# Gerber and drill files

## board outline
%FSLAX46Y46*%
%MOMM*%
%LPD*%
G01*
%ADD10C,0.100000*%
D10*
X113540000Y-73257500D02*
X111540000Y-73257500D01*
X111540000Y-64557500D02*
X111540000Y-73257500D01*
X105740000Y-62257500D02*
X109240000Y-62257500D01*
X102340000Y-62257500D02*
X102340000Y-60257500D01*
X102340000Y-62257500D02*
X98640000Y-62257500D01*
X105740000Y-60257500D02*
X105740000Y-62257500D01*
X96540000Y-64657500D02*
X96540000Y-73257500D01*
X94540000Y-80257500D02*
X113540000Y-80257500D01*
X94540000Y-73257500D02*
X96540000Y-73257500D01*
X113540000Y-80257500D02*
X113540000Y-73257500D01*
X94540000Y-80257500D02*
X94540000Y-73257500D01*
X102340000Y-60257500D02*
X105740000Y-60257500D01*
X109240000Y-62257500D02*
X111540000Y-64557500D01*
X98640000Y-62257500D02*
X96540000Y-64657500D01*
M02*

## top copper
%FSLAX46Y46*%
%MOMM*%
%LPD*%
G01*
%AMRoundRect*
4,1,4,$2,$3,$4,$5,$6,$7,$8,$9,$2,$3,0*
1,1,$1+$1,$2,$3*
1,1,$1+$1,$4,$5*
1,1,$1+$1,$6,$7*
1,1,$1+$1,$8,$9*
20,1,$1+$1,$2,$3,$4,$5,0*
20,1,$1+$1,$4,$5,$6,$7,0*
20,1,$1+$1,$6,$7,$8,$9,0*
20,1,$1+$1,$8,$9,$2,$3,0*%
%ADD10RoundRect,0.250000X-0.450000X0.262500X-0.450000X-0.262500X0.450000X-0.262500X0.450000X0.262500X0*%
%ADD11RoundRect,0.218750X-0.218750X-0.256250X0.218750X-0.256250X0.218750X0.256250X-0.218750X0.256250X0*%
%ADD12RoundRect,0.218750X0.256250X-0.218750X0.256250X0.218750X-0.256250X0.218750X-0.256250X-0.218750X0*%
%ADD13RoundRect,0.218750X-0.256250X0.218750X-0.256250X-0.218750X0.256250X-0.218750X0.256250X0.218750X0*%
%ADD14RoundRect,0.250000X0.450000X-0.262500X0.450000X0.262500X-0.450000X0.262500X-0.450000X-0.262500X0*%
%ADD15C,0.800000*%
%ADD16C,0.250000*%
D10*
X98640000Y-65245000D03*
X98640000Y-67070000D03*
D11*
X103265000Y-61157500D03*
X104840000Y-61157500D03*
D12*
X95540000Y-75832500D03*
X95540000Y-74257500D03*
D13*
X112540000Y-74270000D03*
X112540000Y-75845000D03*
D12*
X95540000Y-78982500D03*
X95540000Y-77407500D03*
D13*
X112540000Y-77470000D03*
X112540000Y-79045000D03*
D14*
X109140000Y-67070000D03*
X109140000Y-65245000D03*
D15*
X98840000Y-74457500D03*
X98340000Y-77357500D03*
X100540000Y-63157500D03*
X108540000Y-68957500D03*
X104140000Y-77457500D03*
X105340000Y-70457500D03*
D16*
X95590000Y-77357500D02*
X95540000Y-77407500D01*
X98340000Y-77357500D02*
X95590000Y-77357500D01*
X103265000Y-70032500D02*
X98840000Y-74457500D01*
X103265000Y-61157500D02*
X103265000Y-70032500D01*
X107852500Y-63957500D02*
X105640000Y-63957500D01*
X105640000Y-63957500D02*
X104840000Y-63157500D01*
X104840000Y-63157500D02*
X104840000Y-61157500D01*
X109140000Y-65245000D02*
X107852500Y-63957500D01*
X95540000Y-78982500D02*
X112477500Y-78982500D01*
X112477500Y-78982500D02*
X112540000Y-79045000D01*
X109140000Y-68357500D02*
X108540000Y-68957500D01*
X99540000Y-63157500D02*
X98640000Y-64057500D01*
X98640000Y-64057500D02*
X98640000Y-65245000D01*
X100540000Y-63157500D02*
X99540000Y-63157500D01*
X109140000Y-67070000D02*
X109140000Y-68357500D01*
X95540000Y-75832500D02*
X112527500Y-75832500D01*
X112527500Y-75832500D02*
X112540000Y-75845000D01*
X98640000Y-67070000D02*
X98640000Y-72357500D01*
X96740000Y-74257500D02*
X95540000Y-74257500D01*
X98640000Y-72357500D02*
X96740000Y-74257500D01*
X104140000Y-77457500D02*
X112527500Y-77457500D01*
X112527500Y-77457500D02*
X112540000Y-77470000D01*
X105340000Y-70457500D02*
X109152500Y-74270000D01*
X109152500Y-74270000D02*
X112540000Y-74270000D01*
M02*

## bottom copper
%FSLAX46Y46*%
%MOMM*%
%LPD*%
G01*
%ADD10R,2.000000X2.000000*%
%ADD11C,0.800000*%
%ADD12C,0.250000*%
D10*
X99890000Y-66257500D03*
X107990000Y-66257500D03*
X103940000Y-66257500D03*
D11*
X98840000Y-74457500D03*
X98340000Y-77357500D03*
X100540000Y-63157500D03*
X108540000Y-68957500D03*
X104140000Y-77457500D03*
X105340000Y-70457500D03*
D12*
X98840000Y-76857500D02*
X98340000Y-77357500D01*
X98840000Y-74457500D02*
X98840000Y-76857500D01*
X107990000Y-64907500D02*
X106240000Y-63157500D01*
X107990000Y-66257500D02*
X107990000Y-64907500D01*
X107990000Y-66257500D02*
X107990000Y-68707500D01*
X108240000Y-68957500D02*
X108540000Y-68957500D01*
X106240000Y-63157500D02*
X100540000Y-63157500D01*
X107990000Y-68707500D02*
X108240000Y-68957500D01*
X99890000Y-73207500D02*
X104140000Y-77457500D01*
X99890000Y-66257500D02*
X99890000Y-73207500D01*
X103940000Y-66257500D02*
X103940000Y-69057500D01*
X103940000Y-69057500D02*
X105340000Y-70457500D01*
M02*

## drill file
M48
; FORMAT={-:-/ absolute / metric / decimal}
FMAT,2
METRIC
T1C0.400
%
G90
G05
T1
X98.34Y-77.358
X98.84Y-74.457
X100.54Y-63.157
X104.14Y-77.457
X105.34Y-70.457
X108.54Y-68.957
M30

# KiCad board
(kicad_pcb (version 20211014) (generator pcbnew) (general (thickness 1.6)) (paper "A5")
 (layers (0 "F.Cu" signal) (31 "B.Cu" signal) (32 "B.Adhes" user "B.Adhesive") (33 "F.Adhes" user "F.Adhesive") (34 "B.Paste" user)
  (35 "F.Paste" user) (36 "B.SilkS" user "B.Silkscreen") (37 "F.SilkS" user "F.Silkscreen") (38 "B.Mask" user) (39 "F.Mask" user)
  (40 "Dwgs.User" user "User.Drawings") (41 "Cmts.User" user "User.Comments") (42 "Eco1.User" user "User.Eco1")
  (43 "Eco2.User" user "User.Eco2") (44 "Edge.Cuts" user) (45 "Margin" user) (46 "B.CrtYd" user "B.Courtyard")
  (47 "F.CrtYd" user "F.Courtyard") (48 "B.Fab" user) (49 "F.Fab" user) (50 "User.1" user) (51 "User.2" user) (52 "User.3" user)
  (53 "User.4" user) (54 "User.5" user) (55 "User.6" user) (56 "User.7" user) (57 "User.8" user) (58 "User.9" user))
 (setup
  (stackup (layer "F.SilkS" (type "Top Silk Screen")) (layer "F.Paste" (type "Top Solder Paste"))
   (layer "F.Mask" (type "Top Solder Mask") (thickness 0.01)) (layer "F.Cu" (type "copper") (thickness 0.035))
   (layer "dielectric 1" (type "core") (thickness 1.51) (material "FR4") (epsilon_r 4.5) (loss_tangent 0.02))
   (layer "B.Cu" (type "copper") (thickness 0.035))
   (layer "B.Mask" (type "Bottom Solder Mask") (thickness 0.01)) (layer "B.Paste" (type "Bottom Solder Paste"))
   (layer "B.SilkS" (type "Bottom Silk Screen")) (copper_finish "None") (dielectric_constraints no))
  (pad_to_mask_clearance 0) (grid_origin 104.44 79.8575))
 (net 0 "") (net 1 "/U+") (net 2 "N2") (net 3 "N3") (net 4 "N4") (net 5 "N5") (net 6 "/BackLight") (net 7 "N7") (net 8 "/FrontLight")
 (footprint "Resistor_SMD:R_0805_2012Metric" (layer "F.Cu") (at 98.64 66.1575 -90)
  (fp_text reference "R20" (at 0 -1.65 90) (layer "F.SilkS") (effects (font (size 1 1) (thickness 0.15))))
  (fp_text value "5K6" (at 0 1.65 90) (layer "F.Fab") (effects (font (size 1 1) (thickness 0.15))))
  (pad "1" smd roundrect locked (at -0.9125 0 270) (size 1.025 1.4) (layers "F.Cu" "F.Paste" "F.Mask") (roundrect_rratio 0.243902439)
   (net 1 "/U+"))
  (pad "2" smd roundrect locked (at 0.9125 0 270) (size 1.025 1.4) (layers "F.Cu" "F.Paste" "F.Mask") (roundrect_rratio 0.243902439)
   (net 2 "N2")))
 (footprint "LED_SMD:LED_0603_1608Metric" (layer "F.Cu") (at 104.0525 61.1575)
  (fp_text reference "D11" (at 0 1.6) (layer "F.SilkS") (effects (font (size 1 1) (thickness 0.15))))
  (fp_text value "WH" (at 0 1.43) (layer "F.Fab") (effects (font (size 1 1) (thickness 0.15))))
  (pad "1" smd roundrect locked (at -0.7875 0) (size 0.875 0.95) (layers "F.Cu" "F.Paste" "F.Mask") (roundrect_rratio 0.25) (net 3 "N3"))
  (pad "2" smd roundrect locked (at 0.7875 0) (size 0.875 0.95) (layers "F.Cu" "F.Paste" "F.Mask") (roundrect_rratio 0.25) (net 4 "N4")))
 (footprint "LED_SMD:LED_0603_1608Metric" (layer "F.Cu") (at 95.54 75.045 90)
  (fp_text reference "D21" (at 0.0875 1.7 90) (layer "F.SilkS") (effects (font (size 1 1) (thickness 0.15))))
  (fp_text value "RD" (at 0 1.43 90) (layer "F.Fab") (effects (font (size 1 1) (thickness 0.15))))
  (pad "1" smd roundrect locked (at -0.7875 0 90) (size 0.875 0.95) (layers "F.Cu" "F.Paste" "F.Mask") (roundrect_rratio 0.25) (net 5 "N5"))
  (pad "2" smd roundrect locked (at 0.7875 0 90) (size 0.875 0.95) (layers "F.Cu" "F.Paste" "F.Mask") (roundrect_rratio 0.25) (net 2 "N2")))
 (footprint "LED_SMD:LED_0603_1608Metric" (layer "F.Cu") (at 112.54 75.0575 -90)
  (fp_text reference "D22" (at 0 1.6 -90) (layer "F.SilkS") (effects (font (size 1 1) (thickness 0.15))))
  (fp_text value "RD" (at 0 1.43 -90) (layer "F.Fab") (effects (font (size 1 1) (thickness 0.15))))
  (pad "1" smd roundrect locked (at -0.7875 0 270) (size 0.875 0.95) (layers "F.Cu" "F.Paste" "F.Mask") (roundrect_rratio 0.25)
   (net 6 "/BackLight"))
  (pad "2" smd roundrect locked (at 0.7875 0 270) (size 0.875 0.95) (layers "F.Cu" "F.Paste" "F.Mask") (roundrect_rratio 0.25) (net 5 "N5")))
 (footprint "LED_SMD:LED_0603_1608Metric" (layer "F.Cu") (at 95.54 78.195 90)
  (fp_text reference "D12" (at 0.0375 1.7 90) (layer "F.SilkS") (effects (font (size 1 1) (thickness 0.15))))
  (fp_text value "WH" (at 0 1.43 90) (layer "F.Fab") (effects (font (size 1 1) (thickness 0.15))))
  (pad "1" smd roundrect locked (at -0.7875 0 90) (size 0.875 0.95) (layers "F.Cu" "F.Paste" "F.Mask") (roundrect_rratio 0.25) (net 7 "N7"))
  (pad "2" smd roundrect locked (at 0.7875 0 90) (size 0.875 0.95) (layers "F.Cu" "F.Paste" "F.Mask") (roundrect_rratio 0.25) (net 3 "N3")))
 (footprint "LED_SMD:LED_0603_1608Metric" (layer "F.Cu") (at 112.54 78.2575 -90)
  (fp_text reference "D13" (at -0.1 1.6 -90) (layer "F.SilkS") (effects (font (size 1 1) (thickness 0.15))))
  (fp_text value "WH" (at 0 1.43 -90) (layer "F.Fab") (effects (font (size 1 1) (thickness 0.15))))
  (pad "1" smd roundrect locked (at -0.7875 0 270) (size 0.875 0.95) (layers "F.Cu" "F.Paste" "F.Mask") (roundrect_rratio 0.25)
   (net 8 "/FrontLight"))
  (pad "2" smd roundrect locked (at 0.7875 0 270) (size 0.875 0.95) (layers "F.Cu" "F.Paste" "F.Mask") (roundrect_rratio 0.25) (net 7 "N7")))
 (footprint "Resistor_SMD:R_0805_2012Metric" (layer "F.Cu") (at 109.14 66.1575 90)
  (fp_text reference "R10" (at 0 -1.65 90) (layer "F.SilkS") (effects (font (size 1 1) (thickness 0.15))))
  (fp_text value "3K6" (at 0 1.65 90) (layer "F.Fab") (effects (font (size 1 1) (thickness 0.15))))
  (pad "1" smd roundrect locked (at -0.9125 0 90) (size 1.025 1.4) (layers "F.Cu" "F.Paste" "F.Mask") (roundrect_rratio 0.243902439)
   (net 1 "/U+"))
  (pad "2" smd roundrect locked (at 0.9125 0 90) (size 1.025 1.4) (layers "F.Cu" "F.Paste" "F.Mask") (roundrect_rratio 0.243902439)
   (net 4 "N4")))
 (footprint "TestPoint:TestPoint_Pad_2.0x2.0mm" (layer "B.Cu") (at 99.89 66.2575 180)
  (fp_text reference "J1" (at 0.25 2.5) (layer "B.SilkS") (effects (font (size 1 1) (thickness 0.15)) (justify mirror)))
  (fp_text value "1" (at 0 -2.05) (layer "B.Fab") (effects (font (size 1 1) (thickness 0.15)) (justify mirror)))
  (pad "1" smd rect locked (at 0 0 180) (size 2 2) (layers "B.Cu" "B.Mask") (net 8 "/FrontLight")))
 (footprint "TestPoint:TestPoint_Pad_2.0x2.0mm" (layer "B.Cu") (at 107.99 66.2575 180)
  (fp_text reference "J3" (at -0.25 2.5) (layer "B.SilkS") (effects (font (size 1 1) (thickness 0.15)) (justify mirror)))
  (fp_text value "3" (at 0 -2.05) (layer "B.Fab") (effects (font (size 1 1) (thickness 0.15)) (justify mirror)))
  (pad "1" smd rect locked (at 0 0 180) (size 2 2) (layers "B.Cu" "B.Mask") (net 1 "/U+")))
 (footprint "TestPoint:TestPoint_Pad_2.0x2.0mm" (layer "B.Cu") (at 103.94 66.2575 180)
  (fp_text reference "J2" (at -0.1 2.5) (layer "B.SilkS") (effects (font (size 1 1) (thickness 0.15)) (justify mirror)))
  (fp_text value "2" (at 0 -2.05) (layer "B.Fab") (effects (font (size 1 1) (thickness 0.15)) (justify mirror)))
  (pad "1" smd rect locked (at 0 0 180) (size 2 2) (layers "B.Cu" "B.Mask") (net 6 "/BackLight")))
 (gr_line (start 113.54 73.2575) (end 111.54 73.2575) (layer "Edge.Cuts") (width 0.1))
 (gr_line (start 111.54 64.5575) (end 111.54 73.2575) (layer "Edge.Cuts") (width 0.1))
 (gr_line (start 105.74 62.2575) (end 109.24 62.2575) (layer "Edge.Cuts") (width 0.1))
 (gr_line (start 102.34 62.2575) (end 102.34 60.2575) (layer "Edge.Cuts") (width 0.1))
 (gr_line (start 102.34 62.2575) (end 98.64 62.2575) (layer "Edge.Cuts") (width 0.1))
 (gr_line (start 105.74 60.2575) (end 105.74 62.2575) (layer "Edge.Cuts") (width 0.1))
 (gr_line (start 96.54 64.6575) (end 96.54 73.2575) (layer "Edge.Cuts") (width 0.1))
 (gr_line (start 94.54 80.2575) (end 113.54 80.2575) (layer "Edge.Cuts") (width 0.1))
 (gr_line (start 94.54 73.2575) (end 96.54 73.2575) (layer "Edge.Cuts") (width 0.1))
 (gr_line (start 113.54 80.2575) (end 113.54 73.2575) (layer "Edge.Cuts") (width 0.1))
 (gr_line (start 94.54 80.2575) (end 94.54 73.2575) (layer "Edge.Cuts") (width 0.1))
 (gr_line (start 102.34 60.2575) (end 105.74 60.2575) (layer "Edge.Cuts") (width 0.1))
 (gr_line (start 109.24 62.2575) (end 111.54 64.5575) (layer "Edge.Cuts") (width 0.1))
 (gr_line (start 98.64 62.2575) (end 96.54 64.6575) (layer "Edge.Cuts") (width 0.1))
 (segment (start 95.59 77.3575) (end 95.54 77.4075) (width 0.25) (layer "F.Cu") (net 3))
 (segment (start 98.34 77.3575) (end 95.59 77.3575) (width 0.25) (layer "F.Cu") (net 3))
 (segment (start 103.265 70.0325) (end 98.84 74.4575) (width 0.25) (layer "F.Cu") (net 3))
 (segment (start 103.265 61.1575) (end 103.265 70.0325) (width 0.25) (layer "F.Cu") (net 3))
 (via (at 98.84 74.4575) (size 0.8) (drill 0.4) (layers "F.Cu" "B.Cu") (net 3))
 (via (at 98.34 77.3575) (size 0.8) (drill 0.4) (layers "F.Cu" "B.Cu") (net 3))
 (segment (start 98.84 76.8575) (end 98.34 77.3575) (width 0.25) (layer "B.Cu") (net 3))
 (segment (start 98.84 74.4575) (end 98.84 76.8575) (width 0.25) (layer "B.Cu") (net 3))
 (segment (start 107.8525 63.9575) (end 105.64 63.9575) (width 0.25) (layer "F.Cu") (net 4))
 (segment (start 105.64 63.9575) (end 104.84 63.1575) (width 0.25) (layer "F.Cu") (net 4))
 (segment (start 104.84 63.1575) (end 104.84 61.1575) (width 0.25) (layer "F.Cu") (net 4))
 (segment (start 109.14 65.245) (end 107.8525 63.9575) (width 0.25) (layer "F.Cu") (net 4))
 (segment (start 95.54 78.9825) (end 112.4775 78.9825) (width 0.25) (layer "F.Cu") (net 7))
 (segment (start 112.4775 78.9825) (end 112.54 79.045) (width 0.25) (layer "F.Cu") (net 7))
 (segment (start 109.14 68.3575) (end 108.54 68.9575) (width 0.25) (layer "F.Cu") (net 1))
 (segment (start 99.54 63.1575) (end 98.64 64.0575) (width 0.25) (layer "F.Cu") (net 1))
 (segment (start 98.64 64.0575) (end 98.64 65.245) (width 0.25) (layer "F.Cu") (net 1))
 (segment (start 100.54 63.1575) (end 99.54 63.1575) (width 0.25) (layer "F.Cu") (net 1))
 (segment (start 109.14 67.07) (end 109.14 68.3575) (width 0.25) (layer "F.Cu") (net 1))
 (via (at 100.54 63.1575) (size 0.8) (drill 0.4) (layers "F.Cu" "B.Cu") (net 1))
 (via (at 108.54 68.9575) (size 0.8) (drill 0.4) (layers "F.Cu" "B.Cu") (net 1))
 (segment (start 107.99 64.9075) (end 106.24 63.1575) (width 0.25) (layer "B.Cu") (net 1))
 (segment (start 107.99 66.2575) (end 107.99 64.9075) (width 0.25) (layer "B.Cu") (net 1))
 (segment (start 107.99 66.2575) (end 107.99 68.7075) (width 0.25) (layer "B.Cu") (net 1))
 (segment (start 108.24 68.9575) (end 108.54 68.9575) (width 0.25) (layer "B.Cu") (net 1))
 (segment (start 106.24 63.1575) (end 100.54 63.1575) (width 0.25) (layer "B.Cu") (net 1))
 (segment (start 107.99 68.7075) (end 108.24 68.9575) (width 0.25) (layer "B.Cu") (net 1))
 (segment (start 95.54 75.8325) (end 112.5275 75.8325) (width 0.25) (layer "F.Cu") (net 5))
 (segment (start 112.5275 75.8325) (end 112.54 75.845) (width 0.25) (layer "F.Cu") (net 5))
 (segment (start 98.64 67.07) (end 98.64 72.3575) (width 0.25) (layer "F.Cu") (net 2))
 (segment (start 96.74 74.2575) (end 95.54 74.2575) (width 0.25) (layer "F.Cu") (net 2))
 (segment (start 98.64 72.3575) (end 96.74 74.2575) (width 0.25) (layer "F.Cu") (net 2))
 (segment (start 104.14 77.4575) (end 112.5275 77.4575) (width 0.25) (layer "F.Cu") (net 8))
 (segment (start 112.5275 77.4575) (end 112.54 77.47) (width 0.25) (layer "F.Cu") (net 8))
 (via (at 104.14 77.4575) (size 0.8) (drill 0.4) (layers "F.Cu" "B.Cu") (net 8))
 (segment (start 99.89 73.2075) (end 104.14 77.4575) (width 0.25) (layer "B.Cu") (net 8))
 (segment (start 99.89 66.2575) (end 99.89 73.2075) (width 0.25) (layer "B.Cu") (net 8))
 (segment (start 105.34 70.4575) (end 109.1525 74.27) (width 0.25) (layer "F.Cu") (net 6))
 (segment (start 109.1525 74.27) (end 112.54 74.27) (width 0.25) (layer "F.Cu") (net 6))
 (via (at 105.34 70.4575) (size 0.8) (drill 0.4) (layers "F.Cu" "B.Cu") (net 6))
 (segment (start 103.94 66.2575) (end 103.94 69.0575) (width 0.25) (layer "B.Cu") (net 6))
 (segment (start 103.94 69.0575) (end 105.34 70.4575) (width 0.25) (layer "B.Cu") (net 6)))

